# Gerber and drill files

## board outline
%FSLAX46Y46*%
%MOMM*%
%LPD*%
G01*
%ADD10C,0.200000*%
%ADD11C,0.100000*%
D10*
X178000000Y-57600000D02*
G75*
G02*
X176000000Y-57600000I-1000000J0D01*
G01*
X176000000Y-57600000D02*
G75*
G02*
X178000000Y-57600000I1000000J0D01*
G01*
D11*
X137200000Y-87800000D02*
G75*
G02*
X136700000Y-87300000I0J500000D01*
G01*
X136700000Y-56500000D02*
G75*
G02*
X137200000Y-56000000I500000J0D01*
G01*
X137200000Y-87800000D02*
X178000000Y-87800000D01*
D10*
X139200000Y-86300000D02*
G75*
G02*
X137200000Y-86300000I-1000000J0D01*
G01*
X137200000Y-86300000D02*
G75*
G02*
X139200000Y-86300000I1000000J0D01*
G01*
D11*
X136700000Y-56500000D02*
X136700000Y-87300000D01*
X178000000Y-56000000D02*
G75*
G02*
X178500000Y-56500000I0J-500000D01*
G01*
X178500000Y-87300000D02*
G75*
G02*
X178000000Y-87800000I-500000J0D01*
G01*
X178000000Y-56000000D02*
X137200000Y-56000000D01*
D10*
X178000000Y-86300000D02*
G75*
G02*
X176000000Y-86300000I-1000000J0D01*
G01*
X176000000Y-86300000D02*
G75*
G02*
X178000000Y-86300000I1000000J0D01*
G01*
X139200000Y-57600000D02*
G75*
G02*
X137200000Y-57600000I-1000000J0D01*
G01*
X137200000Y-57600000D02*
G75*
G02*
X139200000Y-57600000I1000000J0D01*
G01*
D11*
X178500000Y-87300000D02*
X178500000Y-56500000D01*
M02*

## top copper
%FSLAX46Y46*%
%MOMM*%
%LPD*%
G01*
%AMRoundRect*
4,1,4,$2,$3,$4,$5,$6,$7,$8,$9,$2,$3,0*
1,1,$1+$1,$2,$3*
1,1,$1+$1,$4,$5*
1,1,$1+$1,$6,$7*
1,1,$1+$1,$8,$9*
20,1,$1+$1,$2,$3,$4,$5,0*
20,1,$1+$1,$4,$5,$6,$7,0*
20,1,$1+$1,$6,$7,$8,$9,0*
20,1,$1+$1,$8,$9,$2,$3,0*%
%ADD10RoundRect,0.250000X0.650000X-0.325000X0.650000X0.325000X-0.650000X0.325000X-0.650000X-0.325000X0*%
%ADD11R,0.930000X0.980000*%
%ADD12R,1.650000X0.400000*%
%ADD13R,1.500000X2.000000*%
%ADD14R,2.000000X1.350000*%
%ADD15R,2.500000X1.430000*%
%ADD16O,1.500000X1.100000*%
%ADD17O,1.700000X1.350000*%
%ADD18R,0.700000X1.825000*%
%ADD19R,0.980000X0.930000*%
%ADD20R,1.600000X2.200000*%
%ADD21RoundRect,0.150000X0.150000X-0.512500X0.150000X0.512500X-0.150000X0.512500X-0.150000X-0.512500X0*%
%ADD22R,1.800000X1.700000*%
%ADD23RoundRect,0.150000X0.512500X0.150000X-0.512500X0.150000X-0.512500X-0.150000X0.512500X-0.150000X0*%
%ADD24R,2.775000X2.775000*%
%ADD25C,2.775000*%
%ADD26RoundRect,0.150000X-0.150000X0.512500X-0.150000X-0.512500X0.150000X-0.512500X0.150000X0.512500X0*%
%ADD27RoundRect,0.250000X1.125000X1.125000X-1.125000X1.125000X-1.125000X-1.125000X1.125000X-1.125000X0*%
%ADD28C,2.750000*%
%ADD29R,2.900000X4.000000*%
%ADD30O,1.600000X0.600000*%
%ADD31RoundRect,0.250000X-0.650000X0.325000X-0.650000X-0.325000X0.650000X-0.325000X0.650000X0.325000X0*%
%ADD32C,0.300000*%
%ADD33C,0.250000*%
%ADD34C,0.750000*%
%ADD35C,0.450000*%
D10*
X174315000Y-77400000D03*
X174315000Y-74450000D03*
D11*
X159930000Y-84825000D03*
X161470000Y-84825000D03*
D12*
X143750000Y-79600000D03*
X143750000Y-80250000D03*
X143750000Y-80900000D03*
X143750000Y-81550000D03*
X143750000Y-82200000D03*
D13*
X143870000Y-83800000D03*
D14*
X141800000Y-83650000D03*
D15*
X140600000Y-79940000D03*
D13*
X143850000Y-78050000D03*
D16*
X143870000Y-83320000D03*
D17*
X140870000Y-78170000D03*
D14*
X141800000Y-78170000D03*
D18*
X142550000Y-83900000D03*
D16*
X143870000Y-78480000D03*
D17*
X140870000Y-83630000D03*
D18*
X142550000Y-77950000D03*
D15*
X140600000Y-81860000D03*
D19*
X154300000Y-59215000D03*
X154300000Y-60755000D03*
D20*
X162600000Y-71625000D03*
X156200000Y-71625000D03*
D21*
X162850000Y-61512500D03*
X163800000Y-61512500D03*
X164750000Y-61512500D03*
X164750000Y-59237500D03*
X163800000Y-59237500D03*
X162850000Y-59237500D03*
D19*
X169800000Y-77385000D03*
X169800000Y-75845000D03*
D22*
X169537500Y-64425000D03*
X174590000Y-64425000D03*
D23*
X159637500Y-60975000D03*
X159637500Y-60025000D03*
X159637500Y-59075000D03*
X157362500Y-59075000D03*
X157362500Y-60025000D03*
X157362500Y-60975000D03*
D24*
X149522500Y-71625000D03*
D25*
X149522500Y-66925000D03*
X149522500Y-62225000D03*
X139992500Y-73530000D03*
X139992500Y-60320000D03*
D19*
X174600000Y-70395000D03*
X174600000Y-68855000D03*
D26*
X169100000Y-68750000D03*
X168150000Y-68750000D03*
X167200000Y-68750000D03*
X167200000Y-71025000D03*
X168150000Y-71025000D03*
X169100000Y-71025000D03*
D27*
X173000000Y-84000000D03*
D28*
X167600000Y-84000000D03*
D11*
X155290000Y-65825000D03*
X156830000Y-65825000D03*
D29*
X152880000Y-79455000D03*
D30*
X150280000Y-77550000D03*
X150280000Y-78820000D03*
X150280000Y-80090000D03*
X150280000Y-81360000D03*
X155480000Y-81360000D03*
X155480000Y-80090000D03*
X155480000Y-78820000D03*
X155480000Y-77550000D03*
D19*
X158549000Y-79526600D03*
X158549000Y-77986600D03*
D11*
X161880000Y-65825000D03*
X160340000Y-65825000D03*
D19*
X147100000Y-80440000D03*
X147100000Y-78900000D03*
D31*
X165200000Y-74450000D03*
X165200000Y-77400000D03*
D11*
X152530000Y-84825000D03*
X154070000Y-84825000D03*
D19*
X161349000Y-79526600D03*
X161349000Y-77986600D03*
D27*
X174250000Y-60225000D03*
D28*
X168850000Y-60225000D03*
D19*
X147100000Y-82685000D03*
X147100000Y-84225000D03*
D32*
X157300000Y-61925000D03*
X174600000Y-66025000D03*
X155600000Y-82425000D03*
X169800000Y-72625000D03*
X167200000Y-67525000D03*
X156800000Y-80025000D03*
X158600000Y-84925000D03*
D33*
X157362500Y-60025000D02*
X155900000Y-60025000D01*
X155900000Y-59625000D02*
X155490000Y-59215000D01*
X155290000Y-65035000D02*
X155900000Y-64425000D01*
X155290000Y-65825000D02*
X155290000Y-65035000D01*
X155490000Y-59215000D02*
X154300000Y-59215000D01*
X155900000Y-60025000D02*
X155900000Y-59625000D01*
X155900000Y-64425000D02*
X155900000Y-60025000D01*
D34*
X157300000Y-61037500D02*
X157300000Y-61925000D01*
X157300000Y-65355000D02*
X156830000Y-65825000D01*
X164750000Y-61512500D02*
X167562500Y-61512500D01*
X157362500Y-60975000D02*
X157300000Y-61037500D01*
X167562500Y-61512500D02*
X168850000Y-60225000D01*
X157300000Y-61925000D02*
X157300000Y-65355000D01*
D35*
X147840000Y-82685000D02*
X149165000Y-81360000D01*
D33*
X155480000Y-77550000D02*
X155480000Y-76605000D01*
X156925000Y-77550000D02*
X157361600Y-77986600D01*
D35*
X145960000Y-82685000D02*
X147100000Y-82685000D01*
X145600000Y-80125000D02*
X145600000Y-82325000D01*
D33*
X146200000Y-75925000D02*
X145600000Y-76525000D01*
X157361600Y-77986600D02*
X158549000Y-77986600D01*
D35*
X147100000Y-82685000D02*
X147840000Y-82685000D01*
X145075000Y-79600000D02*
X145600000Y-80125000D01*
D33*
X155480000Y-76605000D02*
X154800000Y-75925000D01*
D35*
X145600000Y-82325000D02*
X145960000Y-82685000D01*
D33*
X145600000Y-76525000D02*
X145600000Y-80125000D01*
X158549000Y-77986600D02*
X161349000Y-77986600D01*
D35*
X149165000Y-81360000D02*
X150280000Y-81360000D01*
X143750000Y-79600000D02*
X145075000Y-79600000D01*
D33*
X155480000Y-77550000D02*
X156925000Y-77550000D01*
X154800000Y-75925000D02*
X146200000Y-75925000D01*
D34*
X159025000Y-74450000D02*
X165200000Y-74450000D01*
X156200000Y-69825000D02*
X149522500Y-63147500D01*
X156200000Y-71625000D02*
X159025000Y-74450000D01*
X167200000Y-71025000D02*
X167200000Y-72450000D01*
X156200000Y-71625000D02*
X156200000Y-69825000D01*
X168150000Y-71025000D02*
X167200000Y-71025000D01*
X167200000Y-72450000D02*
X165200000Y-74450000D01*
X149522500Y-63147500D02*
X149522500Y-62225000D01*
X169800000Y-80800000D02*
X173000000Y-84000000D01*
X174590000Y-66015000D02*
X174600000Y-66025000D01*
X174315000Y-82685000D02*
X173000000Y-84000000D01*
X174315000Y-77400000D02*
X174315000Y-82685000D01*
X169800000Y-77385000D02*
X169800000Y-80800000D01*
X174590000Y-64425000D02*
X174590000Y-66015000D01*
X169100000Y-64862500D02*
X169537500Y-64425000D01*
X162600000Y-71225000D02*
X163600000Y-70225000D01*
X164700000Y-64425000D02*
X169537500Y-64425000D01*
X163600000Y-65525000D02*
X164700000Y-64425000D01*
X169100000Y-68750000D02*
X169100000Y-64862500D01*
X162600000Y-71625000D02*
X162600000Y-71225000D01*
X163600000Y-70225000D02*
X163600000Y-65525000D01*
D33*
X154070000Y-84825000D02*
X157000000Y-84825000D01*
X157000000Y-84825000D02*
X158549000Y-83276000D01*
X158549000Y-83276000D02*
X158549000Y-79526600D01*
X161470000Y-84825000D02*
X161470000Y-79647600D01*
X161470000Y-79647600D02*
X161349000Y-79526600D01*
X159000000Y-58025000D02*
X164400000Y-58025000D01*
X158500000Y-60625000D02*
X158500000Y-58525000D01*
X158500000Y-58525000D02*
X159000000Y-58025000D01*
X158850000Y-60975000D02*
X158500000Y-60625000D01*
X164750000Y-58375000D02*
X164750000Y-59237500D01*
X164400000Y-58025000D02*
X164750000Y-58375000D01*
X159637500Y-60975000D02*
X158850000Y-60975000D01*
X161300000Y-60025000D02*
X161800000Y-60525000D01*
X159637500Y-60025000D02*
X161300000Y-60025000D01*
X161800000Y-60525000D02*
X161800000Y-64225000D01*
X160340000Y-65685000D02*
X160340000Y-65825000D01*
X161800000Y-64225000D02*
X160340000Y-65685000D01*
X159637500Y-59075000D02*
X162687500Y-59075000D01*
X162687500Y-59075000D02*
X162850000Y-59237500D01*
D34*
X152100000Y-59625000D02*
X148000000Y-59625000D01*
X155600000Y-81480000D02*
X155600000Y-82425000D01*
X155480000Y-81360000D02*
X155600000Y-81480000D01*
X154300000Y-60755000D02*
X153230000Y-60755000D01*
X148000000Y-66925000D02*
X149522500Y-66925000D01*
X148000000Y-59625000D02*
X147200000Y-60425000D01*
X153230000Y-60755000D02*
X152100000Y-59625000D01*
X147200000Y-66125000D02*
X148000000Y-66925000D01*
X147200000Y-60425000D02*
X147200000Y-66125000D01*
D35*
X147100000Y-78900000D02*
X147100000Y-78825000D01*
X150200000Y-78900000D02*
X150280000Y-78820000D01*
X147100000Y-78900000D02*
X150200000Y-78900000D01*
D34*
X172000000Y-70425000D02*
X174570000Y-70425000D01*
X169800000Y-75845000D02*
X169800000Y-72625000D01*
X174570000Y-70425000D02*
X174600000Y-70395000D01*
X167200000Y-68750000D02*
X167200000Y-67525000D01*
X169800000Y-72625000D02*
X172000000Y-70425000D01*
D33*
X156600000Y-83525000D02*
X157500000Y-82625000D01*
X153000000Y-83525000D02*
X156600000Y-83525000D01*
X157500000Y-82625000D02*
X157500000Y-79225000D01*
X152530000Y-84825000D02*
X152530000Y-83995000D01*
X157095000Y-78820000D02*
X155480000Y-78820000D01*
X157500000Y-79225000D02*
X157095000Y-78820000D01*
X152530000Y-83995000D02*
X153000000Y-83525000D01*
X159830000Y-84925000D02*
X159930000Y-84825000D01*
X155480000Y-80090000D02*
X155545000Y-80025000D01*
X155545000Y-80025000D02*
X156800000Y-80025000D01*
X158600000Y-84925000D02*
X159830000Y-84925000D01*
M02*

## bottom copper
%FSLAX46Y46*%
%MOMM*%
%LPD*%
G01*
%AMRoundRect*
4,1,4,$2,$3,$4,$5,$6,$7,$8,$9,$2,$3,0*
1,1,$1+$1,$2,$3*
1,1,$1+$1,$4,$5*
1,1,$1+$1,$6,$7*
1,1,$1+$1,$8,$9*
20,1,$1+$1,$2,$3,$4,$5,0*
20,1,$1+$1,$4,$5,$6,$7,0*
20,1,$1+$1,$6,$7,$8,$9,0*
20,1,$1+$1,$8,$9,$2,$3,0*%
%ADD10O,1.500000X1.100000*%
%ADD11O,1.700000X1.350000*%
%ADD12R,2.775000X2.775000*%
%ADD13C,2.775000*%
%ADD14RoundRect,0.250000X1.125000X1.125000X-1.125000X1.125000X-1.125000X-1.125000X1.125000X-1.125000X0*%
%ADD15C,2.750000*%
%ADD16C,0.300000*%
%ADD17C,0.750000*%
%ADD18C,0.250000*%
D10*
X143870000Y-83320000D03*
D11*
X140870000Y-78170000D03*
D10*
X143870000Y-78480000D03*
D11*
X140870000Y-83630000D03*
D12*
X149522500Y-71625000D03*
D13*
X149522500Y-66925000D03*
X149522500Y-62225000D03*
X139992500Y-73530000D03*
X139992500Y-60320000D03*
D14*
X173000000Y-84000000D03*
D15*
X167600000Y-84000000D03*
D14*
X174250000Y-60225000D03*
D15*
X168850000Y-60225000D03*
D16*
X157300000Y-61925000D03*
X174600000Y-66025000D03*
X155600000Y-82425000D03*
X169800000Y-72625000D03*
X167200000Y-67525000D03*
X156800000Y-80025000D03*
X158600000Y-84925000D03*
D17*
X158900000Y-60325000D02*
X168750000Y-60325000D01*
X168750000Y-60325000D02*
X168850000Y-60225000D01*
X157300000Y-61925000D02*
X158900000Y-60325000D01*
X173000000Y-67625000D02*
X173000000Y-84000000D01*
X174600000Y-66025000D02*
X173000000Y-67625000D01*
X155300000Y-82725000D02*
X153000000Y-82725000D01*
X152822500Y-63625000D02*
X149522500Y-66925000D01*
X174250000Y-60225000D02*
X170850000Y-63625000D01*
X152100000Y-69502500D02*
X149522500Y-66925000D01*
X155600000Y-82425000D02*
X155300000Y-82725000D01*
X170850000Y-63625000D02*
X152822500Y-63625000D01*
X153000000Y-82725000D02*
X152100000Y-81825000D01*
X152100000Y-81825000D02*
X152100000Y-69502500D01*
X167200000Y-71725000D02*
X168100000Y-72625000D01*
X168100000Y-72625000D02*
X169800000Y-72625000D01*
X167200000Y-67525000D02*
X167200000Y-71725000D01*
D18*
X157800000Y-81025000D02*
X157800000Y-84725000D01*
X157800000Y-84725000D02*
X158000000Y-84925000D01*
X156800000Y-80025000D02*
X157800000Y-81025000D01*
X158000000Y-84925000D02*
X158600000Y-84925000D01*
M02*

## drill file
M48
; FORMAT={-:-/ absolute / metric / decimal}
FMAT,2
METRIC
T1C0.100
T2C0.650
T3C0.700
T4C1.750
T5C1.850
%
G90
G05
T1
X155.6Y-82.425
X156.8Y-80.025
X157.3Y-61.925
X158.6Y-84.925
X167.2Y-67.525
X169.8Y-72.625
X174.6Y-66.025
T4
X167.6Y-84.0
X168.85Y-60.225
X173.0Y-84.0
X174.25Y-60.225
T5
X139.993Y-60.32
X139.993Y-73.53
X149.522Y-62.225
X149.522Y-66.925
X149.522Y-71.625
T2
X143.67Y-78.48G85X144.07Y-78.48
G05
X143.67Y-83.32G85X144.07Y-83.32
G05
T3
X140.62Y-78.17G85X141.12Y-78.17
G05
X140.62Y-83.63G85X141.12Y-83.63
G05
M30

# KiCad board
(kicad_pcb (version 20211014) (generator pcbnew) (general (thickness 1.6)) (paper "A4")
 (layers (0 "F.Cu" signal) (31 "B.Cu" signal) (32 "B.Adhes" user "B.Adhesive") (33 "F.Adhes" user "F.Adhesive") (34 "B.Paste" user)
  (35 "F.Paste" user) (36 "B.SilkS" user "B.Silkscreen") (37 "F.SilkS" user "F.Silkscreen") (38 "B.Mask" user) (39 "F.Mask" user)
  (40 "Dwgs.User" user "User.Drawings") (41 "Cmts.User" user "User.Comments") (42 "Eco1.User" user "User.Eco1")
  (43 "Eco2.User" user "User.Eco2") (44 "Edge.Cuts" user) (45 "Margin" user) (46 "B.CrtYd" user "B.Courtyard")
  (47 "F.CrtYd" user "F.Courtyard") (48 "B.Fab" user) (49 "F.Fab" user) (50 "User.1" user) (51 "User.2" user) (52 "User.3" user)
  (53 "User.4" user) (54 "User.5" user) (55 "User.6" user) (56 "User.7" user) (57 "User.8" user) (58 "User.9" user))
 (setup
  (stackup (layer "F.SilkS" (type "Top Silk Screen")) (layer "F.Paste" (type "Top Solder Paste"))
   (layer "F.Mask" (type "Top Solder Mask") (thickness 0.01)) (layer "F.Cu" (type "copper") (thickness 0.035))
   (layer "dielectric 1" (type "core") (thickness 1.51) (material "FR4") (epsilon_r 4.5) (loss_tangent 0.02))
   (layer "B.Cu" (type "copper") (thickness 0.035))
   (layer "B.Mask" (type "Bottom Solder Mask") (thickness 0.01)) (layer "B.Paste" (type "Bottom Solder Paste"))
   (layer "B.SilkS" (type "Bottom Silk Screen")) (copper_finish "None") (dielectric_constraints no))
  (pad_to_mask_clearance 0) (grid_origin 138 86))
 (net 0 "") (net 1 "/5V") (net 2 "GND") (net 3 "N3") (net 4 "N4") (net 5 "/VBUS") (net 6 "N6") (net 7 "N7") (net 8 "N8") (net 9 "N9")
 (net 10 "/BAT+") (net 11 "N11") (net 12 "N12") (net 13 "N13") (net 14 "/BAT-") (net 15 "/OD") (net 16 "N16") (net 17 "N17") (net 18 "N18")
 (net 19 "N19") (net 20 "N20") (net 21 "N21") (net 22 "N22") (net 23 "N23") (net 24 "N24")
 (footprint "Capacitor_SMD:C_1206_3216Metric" (layer "F.Cu") (at 174.315 75.925 90)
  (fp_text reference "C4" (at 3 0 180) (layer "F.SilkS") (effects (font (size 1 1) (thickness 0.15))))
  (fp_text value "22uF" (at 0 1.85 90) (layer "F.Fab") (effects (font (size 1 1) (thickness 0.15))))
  (pad "1" smd roundrect (at -1.475 0 90) (size 1.15 1.8) (layers "F.Cu" "F.Paste" "F.Mask") (roundrect_rratio 0.217391) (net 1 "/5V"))
  (pad "2" smd roundrect (at 1.475 0 90) (size 1.15 1.8) (layers "F.Cu" "F.Paste" "F.Mask") (roundrect_rratio 0.217391) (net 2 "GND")))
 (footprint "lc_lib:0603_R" (layer "F.Cu") (at 160.7 84.825)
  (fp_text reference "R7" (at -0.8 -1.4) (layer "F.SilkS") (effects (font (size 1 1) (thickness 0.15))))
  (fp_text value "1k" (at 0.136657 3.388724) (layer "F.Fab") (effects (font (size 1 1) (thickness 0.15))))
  (pad "1" smd rect locked (at -0.77 0) (size 0.93 0.98) (layers "F.Cu" "F.Paste" "F.Mask") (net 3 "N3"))
  (pad "2" smd rect locked (at 0.77 0) (size 0.93 0.98) (layers "F.Cu" "F.Paste" "F.Mask") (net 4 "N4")))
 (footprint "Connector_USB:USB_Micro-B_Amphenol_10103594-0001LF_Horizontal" (layer "F.Cu") (at 141.985 80.925 -90)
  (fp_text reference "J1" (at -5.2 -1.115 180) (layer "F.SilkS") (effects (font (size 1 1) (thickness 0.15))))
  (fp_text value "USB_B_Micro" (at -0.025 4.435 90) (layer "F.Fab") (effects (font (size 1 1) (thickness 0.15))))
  (pad "1" smd rect (at -1.325 -1.765) (size 1.65 0.4) (layers "F.Cu" "F.Paste" "F.Mask") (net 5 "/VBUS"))
  (pad "2" smd rect (at -0.675 -1.765) (size 1.65 0.4) (layers "F.Cu" "F.Paste" "F.Mask") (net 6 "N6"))
  (pad "3" smd rect (at -0.025 -1.765) (size 1.65 0.4) (layers "F.Cu" "F.Paste" "F.Mask") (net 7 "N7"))
  (pad "4" smd rect (at 0.625 -1.765) (size 1.65 0.4) (layers "F.Cu" "F.Paste" "F.Mask") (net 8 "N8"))
  (pad "5" smd rect (at 1.275 -1.765) (size 1.65 0.4) (layers "F.Cu" "F.Paste" "F.Mask") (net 2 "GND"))
  (pad "6" smd rect (at 2.875 -1.885 270) (size 2 1.5) (layers "F.Cu" "F.Paste" "F.Mask") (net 2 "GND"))
  (pad "6" smd rect (at 2.725 0.185 270) (size 1.35 2) (layers "F.Cu" "F.Paste" "F.Mask") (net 2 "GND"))
  (pad "6" smd rect (at -0.985 1.385) (size 2.5 1.43) (layers "F.Cu" "F.Paste" "F.Mask") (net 2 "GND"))
  (pad "6" smd rect (at -2.875 -1.865 270) (size 2 1.5) (layers "F.Cu" "F.Paste" "F.Mask") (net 2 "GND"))
  (pad "6" thru_hole oval (at 2.395 -1.885) (size 1.5 1.1) (drill oval 1.05 0.65) (layers *.Cu *.Mask) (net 2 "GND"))
  (pad "6" thru_hole oval (at -2.755 1.115) (size 1.7 1.35) (drill oval 1.2 0.7) (layers *.Cu *.Mask) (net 2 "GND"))
  (pad "6" smd rect (at -2.755 0.185 270) (size 1.35 2) (layers "F.Cu" "F.Paste" "F.Mask") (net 2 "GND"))
  (pad "6" smd rect (at 2.975 -0.565 270) (size 1.825 0.7) (layers "F.Cu" "F.Paste" "F.Mask") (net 2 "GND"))
  (pad "6" thru_hole oval (at -2.445 -1.885) (size 1.5 1.1) (drill oval 1.05 0.65) (layers *.Cu *.Mask) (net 2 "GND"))
  (pad "6" thru_hole oval (at 2.705 1.115) (size 1.7 1.35) (drill oval 1.2 0.7) (layers *.Cu *.Mask) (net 2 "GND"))
  (pad "6" smd rect (at -2.975 -0.565 270) (size 1.825 0.7) (layers "F.Cu" "F.Paste" "F.Mask") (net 2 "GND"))
  (pad "6" smd rect (at 0.935 1.385) (size 2.5 1.43) (layers "F.Cu" "F.Paste" "F.Mask") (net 2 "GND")))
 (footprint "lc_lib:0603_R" (layer "F.Cu") (at 154.3 59.985 -90)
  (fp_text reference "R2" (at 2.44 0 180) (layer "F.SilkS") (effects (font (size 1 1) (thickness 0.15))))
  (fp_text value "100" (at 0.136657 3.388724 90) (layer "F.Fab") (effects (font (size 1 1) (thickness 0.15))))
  (pad "1" smd rect locked (at -0.77 0 270) (size 0.93 0.98) (layers "F.Cu" "F.Paste" "F.Mask") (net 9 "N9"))
  (pad "2" smd rect locked (at 0.77 0 270) (size 0.93 0.98) (layers "F.Cu" "F.Paste" "F.Mask") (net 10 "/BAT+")))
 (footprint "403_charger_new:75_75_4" (layer "F.Cu") (at 163.15 67.625 180)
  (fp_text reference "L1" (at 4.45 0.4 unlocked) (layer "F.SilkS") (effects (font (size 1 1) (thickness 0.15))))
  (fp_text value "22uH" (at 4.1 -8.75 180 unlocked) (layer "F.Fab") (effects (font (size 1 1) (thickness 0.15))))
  (pad "1" smd rect (at 0.55 -4 90) (size 2.2 1.6) (layers "F.Cu" "F.Paste" "F.Mask") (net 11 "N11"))
  (pad "2" smd rect (at 6.95 -4 90) (size 2.2 1.6) (layers "F.Cu" "F.Adhes" "F.Paste" "F.Mask") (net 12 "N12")))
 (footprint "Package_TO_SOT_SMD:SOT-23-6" (layer "F.Cu") (at 163.8 60.375 90)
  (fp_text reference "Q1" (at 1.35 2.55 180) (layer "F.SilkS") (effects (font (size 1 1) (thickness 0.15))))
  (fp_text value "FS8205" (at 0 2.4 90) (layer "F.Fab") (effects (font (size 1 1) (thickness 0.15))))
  (pad "1" smd roundrect (at -1.1375 -0.95 90) (size 1.325 0.6) (layers "F.Cu" "F.Paste" "F.Mask") (roundrect_rratio 0.25) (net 2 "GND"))
  (pad "2" smd roundrect (at -1.1375 0 90) (size 1.325 0.6) (layers "F.Cu" "F.Paste" "F.Mask") (roundrect_rratio 0.25) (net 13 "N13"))
  (pad "3" smd roundrect (at -1.1375 0.95 90) (size 1.325 0.6) (layers "F.Cu" "F.Paste" "F.Mask") (roundrect_rratio 0.25) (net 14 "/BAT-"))
  (pad "4" smd roundrect (at 1.1375 0.95 90) (size 1.325 0.6) (layers "F.Cu" "F.Paste" "F.Mask") (roundrect_rratio 0.25) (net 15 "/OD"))
  (pad "5" smd roundrect (at 1.1375 0 90) (size 1.325 0.6) (layers "F.Cu" "F.Paste" "F.Mask") (roundrect_rratio 0.25) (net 13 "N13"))
  (pad "6" smd roundrect (at 1.1375 -0.95 90) (size 1.325 0.6) (layers "F.Cu" "F.Paste" "F.Mask") (roundrect_rratio 0.25) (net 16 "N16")))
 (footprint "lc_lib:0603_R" (layer "F.Cu") (at 169.8 76.615 90)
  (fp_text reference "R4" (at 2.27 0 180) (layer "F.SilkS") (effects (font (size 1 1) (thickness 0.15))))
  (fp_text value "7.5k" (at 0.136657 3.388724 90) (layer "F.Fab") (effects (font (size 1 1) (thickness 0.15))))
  (pad "1" smd rect locked (at -0.77 0 90) (size 0.93 0.98) (layers "F.Cu" "F.Paste" "F.Mask") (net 1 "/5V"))
  (pad "2" smd rect locked (at 0.77 0 90) (size 0.93 0.98) (layers "F.Cu" "F.Paste" "F.Mask") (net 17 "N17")))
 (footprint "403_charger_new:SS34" (layer "F.Cu") (at 172.06375 64.425 180)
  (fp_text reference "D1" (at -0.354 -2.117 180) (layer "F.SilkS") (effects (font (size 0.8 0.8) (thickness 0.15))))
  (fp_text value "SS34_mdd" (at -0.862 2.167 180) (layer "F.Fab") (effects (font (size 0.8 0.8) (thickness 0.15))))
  (pad "A" smd rect (at 2.52625 0 180) (size 1.8 1.7) (layers "F.Cu" "F.Paste" "F.Mask") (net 11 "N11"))
  (pad "C" smd rect (at -2.52625 0 180) (size 1.8 1.7) (layers "F.Cu" "F.Paste" "F.Mask") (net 1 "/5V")))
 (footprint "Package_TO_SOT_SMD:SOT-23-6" (layer "F.Cu") (at 158.5 60.025 180)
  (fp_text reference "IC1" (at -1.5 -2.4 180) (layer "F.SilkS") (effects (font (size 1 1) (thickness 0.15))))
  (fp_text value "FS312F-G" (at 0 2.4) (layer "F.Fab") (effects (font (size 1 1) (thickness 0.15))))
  (pad "1" smd roundrect (at -1.1375 -0.95 180) (size 1.325 0.6) (layers "F.Cu" "F.Paste" "F.Mask") (roundrect_rratio 0.25) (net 15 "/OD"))
  (pad "2" smd roundrect (at -1.1375 0 180) (size 1.325 0.6) (layers "F.Cu" "F.Paste" "F.Mask") (roundrect_rratio 0.25) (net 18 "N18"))
  (pad "3" smd roundrect (at -1.1375 0.95 180) (size 1.325 0.6) (layers "F.Cu" "F.Paste" "F.Mask") (roundrect_rratio 0.25) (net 16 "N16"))
  (pad "4" smd roundrect (at 1.1375 0.95 180) (size 1.325 0.6) (layers "F.Cu" "F.Paste" "F.Mask") (roundrect_rratio 0.25) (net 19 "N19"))
  (pad "5" smd roundrect (at 1.1375 0 180) (size 1.325 0.6) (layers "F.Cu" "F.Paste" "F.Mask") (roundrect_rratio 0.25) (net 9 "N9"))
  (pad "6" smd roundrect (at 1.1375 -0.95 180) (size 1.325 0.6) (layers "F.Cu" "F.Paste" "F.Mask") (roundrect_rratio 0.25) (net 14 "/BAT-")))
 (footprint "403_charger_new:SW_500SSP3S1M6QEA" (layer "F.Cu") (at 144.7575 66.925 90)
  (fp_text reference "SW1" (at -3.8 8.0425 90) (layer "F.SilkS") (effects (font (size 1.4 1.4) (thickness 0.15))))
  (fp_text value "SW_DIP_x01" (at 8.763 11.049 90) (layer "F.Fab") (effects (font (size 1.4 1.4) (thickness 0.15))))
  (pad "1" thru_hole rect (at -4.7 4.765 90) (size 2.775 2.775) (drill 1.85) (layers *.Cu *.Mask) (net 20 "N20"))
  (pad "2" thru_hole circle (at 0 4.765 90) (size 2.775 2.775) (drill 1.85) (layers *.Cu *.Mask) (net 10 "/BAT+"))
  (pad "3" thru_hole circle (at 4.7 4.765 90) (size 2.775 2.775) (drill 1.85) (layers *.Cu *.Mask) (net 12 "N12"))
  (pad "S1" thru_hole circle (at -6.605 -4.765 90) (size 2.775 2.775) (drill 1.85) (layers *.Cu *.Mask))
  (pad "S2" thru_hole circle (at 6.605 -4.765 90) (size 2.775 2.775) (drill 1.85) (layers *.Cu *.Mask)))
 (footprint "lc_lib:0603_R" (layer "F.Cu") (at 174.6 69.625 90)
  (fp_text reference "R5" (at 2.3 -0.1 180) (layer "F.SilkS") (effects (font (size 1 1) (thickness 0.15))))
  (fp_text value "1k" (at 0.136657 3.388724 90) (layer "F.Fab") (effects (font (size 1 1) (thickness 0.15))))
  (pad "1" smd rect locked (at -0.77 0 90) (size 0.93 0.98) (layers "F.Cu" "F.Paste" "F.Mask") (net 17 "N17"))
  (pad "2" smd rect locked (at 0.77 0 90) (size 0.93 0.98) (layers "F.Cu" "F.Paste" "F.Mask") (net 2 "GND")))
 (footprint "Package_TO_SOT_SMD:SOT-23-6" (layer "F.Cu") (at 168.15 69.8875 -90)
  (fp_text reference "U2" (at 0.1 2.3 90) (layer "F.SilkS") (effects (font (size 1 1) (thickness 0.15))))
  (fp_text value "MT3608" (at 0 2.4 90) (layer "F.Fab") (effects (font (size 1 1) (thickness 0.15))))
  (pad "1" smd roundrect (at -1.1375 -0.95 270) (size 1.325 0.6) (layers "F.Cu" "F.Paste" "F.Mask") (roundrect_rratio 0.25) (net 11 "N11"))
  (pad "2" smd roundrect (at -1.1375 0 270) (size 1.325 0.6) (layers "F.Cu" "F.Paste" "F.Mask") (roundrect_rratio 0.25) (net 2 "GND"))
  (pad "3" smd roundrect (at -1.1375 0.95 270) (size 1.325 0.6) (layers "F.Cu" "F.Paste" "F.Mask") (roundrect_rratio 0.25) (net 17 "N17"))
  (pad "4" smd roundrect (at 1.1375 0.95 270) (size 1.325 0.6) (layers "F.Cu" "F.Paste" "F.Mask") (roundrect_rratio 0.25) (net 12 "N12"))
  (pad "5" smd roundrect (at 1.1375 0 270) (size 1.325 0.6) (layers "F.Cu" "F.Paste" "F.Mask") (roundrect_rratio 0.25) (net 12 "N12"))
  (pad "6" smd roundrect (at 1.1375 -0.95 270) (size 1.325 0.6) (layers "F.Cu" "F.Paste" "F.Mask") (roundrect_rratio 0.25) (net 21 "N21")))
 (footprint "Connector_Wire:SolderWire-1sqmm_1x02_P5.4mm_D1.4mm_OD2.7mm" (layer "F.Cu") (at 173 84 180)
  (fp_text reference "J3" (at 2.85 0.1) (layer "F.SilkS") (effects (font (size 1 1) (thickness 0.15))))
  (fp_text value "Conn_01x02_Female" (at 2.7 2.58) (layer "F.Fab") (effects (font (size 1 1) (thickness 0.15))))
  (pad "1" thru_hole roundrect (at 0 0 180) (size 2.75 2.75) (drill 1.75) (layers *.Cu *.Mask) (roundrect_rratio 0.090909) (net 1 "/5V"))
  (pad "2" thru_hole circle (at 5.4 0 180) (size 2.75 2.75) (drill 1.75) (layers *.Cu *.Mask) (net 2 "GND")))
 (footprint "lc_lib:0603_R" (layer "F.Cu") (at 156.06 65.825)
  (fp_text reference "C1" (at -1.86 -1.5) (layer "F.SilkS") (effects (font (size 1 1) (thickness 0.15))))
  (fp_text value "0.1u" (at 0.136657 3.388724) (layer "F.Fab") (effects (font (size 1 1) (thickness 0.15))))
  (pad "1" smd rect locked (at -0.77 0) (size 0.93 0.98) (layers "F.Cu" "F.Paste" "F.Mask") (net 9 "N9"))
  (pad "2" smd rect locked (at 0.77 0) (size 0.93 0.98) (layers "F.Cu" "F.Paste" "F.Mask") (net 14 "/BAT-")))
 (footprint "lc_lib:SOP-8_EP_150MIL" (layer "F.Cu") (at 152.88 79.455 -90)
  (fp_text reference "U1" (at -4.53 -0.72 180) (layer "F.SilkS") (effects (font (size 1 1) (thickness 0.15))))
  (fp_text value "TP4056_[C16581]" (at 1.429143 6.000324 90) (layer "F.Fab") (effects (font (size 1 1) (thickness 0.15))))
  (pad "0" smd rect (at 0 0 90) (size 4 2.9) (layers "F.Cu" "F.Paste" "F.Mask"))
  (pad "1" smd oval (at -1.905 2.6 90) (size 0.6 1.6) (layers "F.Cu" "F.Paste" "F.Mask") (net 2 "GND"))
  (pad "2" smd oval (at -0.635 2.6 90) (size 0.6 1.6) (layers "F.Cu" "F.Paste" "F.Mask") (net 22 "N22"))
  (pad "3" smd oval (at 0.635 2.6 90) (size 0.6 1.6) (layers "F.Cu" "F.Paste" "F.Mask") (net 2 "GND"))
  (pad "4" smd oval (at 1.905 2.6 90) (size 0.6 1.6) (layers "F.Cu" "F.Paste" "F.Mask") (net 5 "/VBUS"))
  (pad "5" smd oval (at 1.905 -2.6 90) (size 0.6 1.6) (layers "F.Cu" "F.Paste" "F.Mask") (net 10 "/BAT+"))
  (pad "6" smd oval (at 0.635 -2.6 90) (size 0.6 1.6) (layers "F.Cu" "F.Paste" "F.Mask") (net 3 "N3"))
  (pad "7" smd oval (at -0.635 -2.6 90) (size 0.6 1.6) (layers "F.Cu" "F.Paste" "F.Mask") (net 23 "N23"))
  (pad "8" smd oval (at -1.905 -2.6 90) (size 0.6 1.6) (layers "F.Cu" "F.Paste" "F.Mask") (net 5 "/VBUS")))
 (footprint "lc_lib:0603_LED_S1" (layer "F.Cu") (at 158.549 78.7566 -90)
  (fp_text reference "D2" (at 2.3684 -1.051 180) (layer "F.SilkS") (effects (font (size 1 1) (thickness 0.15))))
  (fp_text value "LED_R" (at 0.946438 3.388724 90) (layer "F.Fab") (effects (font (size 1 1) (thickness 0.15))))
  (pad "1" smd rect (at 0.77 0 90) (size 0.93 0.98) (layers "F.Cu" "F.Paste" "F.Mask") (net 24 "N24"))
  (pad "2" smd rect (at -0.77 0 90) (size 0.93 0.98) (layers "F.Cu" "F.Paste" "F.Mask") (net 5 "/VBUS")))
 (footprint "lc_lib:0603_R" (layer "F.Cu") (at 161.11 65.825 180)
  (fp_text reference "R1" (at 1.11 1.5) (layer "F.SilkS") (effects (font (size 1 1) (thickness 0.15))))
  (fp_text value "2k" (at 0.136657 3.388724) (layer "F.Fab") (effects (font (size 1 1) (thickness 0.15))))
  (pad "1" smd rect locked (at -0.77 0 180) (size 0.93 0.98) (layers "F.Cu" "F.Paste" "F.Mask") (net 2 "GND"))
  (pad "2" smd rect locked (at 0.77 0 180) (size 0.93 0.98) (layers "F.Cu" "F.Paste" "F.Mask") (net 18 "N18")))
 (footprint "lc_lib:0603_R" (layer "F.Cu") (at 147.1 79.67 90)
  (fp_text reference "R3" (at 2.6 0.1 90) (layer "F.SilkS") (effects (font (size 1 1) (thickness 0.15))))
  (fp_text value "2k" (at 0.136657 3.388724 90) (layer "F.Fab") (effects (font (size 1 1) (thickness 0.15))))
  (pad "1" smd rect locked (at -0.77 0 90) (size 0.93 0.98) (layers "F.Cu" "F.Paste" "F.Mask") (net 2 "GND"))
  (pad "2" smd rect locked (at 0.77 0 90) (size 0.93 0.98) (layers "F.Cu" "F.Paste" "F.Mask") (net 22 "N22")))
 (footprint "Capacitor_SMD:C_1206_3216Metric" (layer "F.Cu") (at 165.2 75.925 -90)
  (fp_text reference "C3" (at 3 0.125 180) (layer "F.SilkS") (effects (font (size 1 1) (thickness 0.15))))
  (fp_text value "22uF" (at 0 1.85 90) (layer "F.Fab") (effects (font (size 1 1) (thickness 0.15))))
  (pad "1" smd roundrect (at -1.475 0 270) (size 1.15 1.8) (layers "F.Cu" "F.Paste" "F.Mask") (roundrect_rratio 0.217391) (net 12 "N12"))
  (pad "2" smd roundrect (at 1.475 0 270) (size 1.15 1.8) (layers "F.Cu" "F.Paste" "F.Mask") (roundrect_rratio 0.217391) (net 2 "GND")))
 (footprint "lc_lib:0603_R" (layer "F.Cu") (at 153.3 84.825)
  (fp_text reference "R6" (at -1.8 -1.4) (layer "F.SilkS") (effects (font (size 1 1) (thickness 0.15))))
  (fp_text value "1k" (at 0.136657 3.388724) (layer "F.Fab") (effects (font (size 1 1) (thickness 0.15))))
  (pad "1" smd rect locked (at -0.77 0) (size 0.93 0.98) (layers "F.Cu" "F.Paste" "F.Mask") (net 23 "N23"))
  (pad "2" smd rect locked (at 0.77 0) (size 0.93 0.98) (layers "F.Cu" "F.Paste" "F.Mask") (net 24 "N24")))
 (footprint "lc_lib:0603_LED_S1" (layer "F.Cu") (at 161.349 78.7566 -90)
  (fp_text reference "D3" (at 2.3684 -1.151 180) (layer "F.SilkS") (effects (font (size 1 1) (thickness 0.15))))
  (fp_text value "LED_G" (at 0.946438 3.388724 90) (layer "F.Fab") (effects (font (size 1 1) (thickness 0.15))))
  (pad "1" smd rect (at 0.77 0 90) (size 0.93 0.98) (layers "F.Cu" "F.Paste" "F.Mask") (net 4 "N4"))
  (pad "2" smd rect (at -0.77 0 90) (size 0.93 0.98) (layers "F.Cu" "F.Paste" "F.Mask") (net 5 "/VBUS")))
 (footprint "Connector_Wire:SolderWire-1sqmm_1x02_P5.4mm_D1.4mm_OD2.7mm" (layer "F.Cu") (at 174.25 60.225 180)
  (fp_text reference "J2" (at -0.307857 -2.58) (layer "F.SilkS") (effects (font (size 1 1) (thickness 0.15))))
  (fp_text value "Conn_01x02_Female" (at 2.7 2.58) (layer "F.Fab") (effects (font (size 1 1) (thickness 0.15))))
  (pad "1" thru_hole roundrect (at 0 0 180) (size 2.75 2.75) (drill 1.75) (layers *.Cu *.Mask) (roundrect_rratio 0.090909) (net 10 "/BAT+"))
  (pad "2" thru_hole circle (at 5.4 0 180) (size 2.75 2.75) (drill 1.75) (layers *.Cu *.Mask) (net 14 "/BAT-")))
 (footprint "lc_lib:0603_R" (layer "F.Cu") (at 147.1 83.455 -90)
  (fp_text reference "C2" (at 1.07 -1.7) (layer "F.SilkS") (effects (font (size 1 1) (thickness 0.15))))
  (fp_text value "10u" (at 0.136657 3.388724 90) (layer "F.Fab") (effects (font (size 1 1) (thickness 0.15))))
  (pad "1" smd rect locked (at -0.77 0 270) (size 0.93 0.98) (layers "F.Cu" "F.Paste" "F.Mask") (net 5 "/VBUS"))
  (pad "2" smd rect locked (at 0.77 0 270) (size 0.93 0.98) (layers "F.Cu" "F.Paste" "F.Mask") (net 2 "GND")))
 (gr_circle (center 177 57.6) (end 178 57.6) (layer "Edge.Cuts") (width 0.2) (fill none))
 (gr_arc (start 137.2 87.8) (mid 136.846447 87.653553) (end 136.7 87.3) (layer "Edge.Cuts") (width 0.1))
 (gr_arc (start 136.7 56.5) (mid 136.846447 56.146447) (end 137.2 56) (layer "Edge.Cuts") (width 0.1))
 (gr_line (start 137.2 87.8) (end 178 87.8) (layer "Edge.Cuts") (width 0.1))
 (gr_circle (center 138.2 86.3) (end 138.2 85.3) (layer "Edge.Cuts") (width 0.2) (fill none))
 (gr_line (start 136.7 56.5) (end 136.7 87.3) (layer "Edge.Cuts") (width 0.1))
 (gr_arc (start 178 56) (mid 178.353553 56.146447) (end 178.5 56.5) (layer "Edge.Cuts") (width 0.1))
 (gr_arc (start 178.5 87.3) (mid 178.353553 87.653553) (end 178 87.8) (layer "Edge.Cuts") (width 0.1))
 (gr_line (start 178 56) (end 137.2 56) (layer "Edge.Cuts") (width 0.1))
 (gr_circle (center 177 86.3) (end 177 85.3) (layer "Edge.Cuts") (width 0.2) (fill none))
 (gr_circle (center 138.2 57.6) (end 138.2 56.6) (layer "Edge.Cuts") (width 0.2) (fill none))
 (gr_line (start 178.5 87.3) (end 178.5 56.5) (layer "Edge.Cuts") (width 0.1))
 (segment (start 157.3625 60.025) (end 155.9 60.025) (width 0.25) (layer "F.Cu") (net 9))
 (segment (start 155.9 59.625) (end 155.49 59.215) (width 0.25) (layer "F.Cu") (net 9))
 (segment (start 155.29 65.035) (end 155.9 64.425) (width 0.25) (layer "F.Cu") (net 9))
 (segment (start 155.29 65.825) (end 155.29 65.035) (width 0.25) (layer "F.Cu") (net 9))
 (segment (start 155.49 59.215) (end 154.3 59.215) (width 0.25) (layer "F.Cu") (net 9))
 (segment (start 155.9 60.025) (end 155.9 59.625) (width 0.25) (layer "F.Cu") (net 9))
 (segment (start 155.9 64.425) (end 155.9 60.025) (width 0.25) (layer "F.Cu") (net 9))
 (segment (start 157.3 61.0375) (end 157.3 61.925) (width 0.75) (layer "F.Cu") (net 14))
 (segment (start 157.3 65.355) (end 156.83 65.825) (width 0.75) (layer "F.Cu") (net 14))
 (segment (start 164.75 61.5125) (end 167.5625 61.5125) (width 0.75) (layer "F.Cu") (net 14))
 (segment (start 157.3625 60.975) (end 157.3 61.0375) (width 0.75) (layer "F.Cu") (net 14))
 (segment (start 167.5625 61.5125) (end 168.85 60.225) (width 0.75) (layer "F.Cu") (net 14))
 (segment (start 157.3 61.925) (end 157.3 65.355) (width 0.75) (layer "F.Cu") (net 14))
 (via micro (at 157.3 61.925) (size 0.3) (drill 0.1) (layers "F.Cu" "B.Cu") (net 14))
 (segment (start 158.9 60.325) (end 168.75 60.325) (width 0.75) (layer "B.Cu") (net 14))
 (segment (start 168.75 60.325) (end 168.85 60.225) (width 0.75) (layer "B.Cu") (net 14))
 (segment (start 157.3 61.925) (end 158.9 60.325) (width 0.75) (layer "B.Cu") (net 14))
 (segment (start 147.84 82.685) (end 149.165 81.36) (width 0.45) (layer "F.Cu") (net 5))
 (segment (start 155.48 77.55) (end 155.48 76.605) (width 0.25) (layer "F.Cu") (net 5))
 (segment (start 156.925 77.55) (end 157.3616 77.9866) (width 0.25) (layer "F.Cu") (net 5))
 (segment (start 145.96 82.685) (end 147.1 82.685) (width 0.45) (layer "F.Cu") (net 5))
 (segment (start 145.6 80.125) (end 145.6 82.325) (width 0.45) (layer "F.Cu") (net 5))
 (segment (start 146.2 75.925) (end 145.6 76.525) (width 0.25) (layer "F.Cu") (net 5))
 (segment (start 157.3616 77.9866) (end 158.549 77.9866) (width 0.25) (layer "F.Cu") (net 5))
 (segment (start 147.1 82.685) (end 147.84 82.685) (width 0.45) (layer "F.Cu") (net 5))
 (segment (start 145.075 79.6) (end 145.6 80.125) (width 0.45) (layer "F.Cu") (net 5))
 (segment (start 155.48 76.605) (end 154.8 75.925) (width 0.25) (layer "F.Cu") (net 5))
 (segment (start 145.6 82.325) (end 145.96 82.685) (width 0.45) (layer "F.Cu") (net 5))
 (segment (start 145.6 76.525) (end 145.6 80.125) (width 0.25) (layer "F.Cu") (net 5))
 (segment (start 158.549 77.9866) (end 161.349 77.9866) (width 0.25) (layer "F.Cu") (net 5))
 (segment (start 149.165 81.36) (end 150.28 81.36) (width 0.45) (layer "F.Cu") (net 5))
 (segment (start 143.75 79.6) (end 145.075 79.6) (width 0.45) (layer "F.Cu") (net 5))
 (segment (start 155.48 77.55) (end 156.925 77.55) (width 0.25) (layer "F.Cu") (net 5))
 (segment (start 154.8 75.925) (end 146.2 75.925) (width 0.25) (layer "F.Cu") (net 5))
 (segment (start 159.025 74.45) (end 165.2 74.45) (width 0.75) (layer "F.Cu") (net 12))
 (segment (start 156.2 69.825) (end 149.5225 63.1475) (width 0.75) (layer "F.Cu") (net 12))
 (segment (start 156.2 71.625) (end 159.025 74.45) (width 0.75) (layer "F.Cu") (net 12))
 (segment (start 167.2 71.025) (end 167.2 72.45) (width 0.75) (layer "F.Cu") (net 12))
 (segment (start 156.2 71.625) (end 156.2 69.825) (width 0.75) (layer "F.Cu") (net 12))
 (segment (start 168.15 71.025) (end 167.2 71.025) (width 0.75) (layer "F.Cu") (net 12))
 (segment (start 167.2 72.45) (end 165.2 74.45) (width 0.75) (layer "F.Cu") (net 12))
 (segment (start 149.5225 63.1475) (end 149.5225 62.225) (width 0.75) (layer "F.Cu") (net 12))
 (segment (start 169.8 80.8) (end 173 84) (width 0.75) (layer "F.Cu") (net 1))
 (segment (start 174.59 66.015) (end 174.6 66.025) (width 0.75) (layer "F.Cu") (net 1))
 (segment (start 174.315 82.685) (end 173 84) (width 0.75) (layer "F.Cu") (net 1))
 (segment (start 174.315 77.4) (end 174.315 82.685) (width 0.75) (layer "F.Cu") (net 1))
 (segment (start 169.8 77.385) (end 169.8 80.8) (width 0.75) (layer "F.Cu") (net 1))
 (segment (start 174.59 64.425) (end 174.59 66.015) (width 0.75) (layer "F.Cu") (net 1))
 (via micro (at 174.6 66.025) (size 0.3) (drill 0.1) (layers "F.Cu" "B.Cu") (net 1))
 (segment (start 173 67.625) (end 173 84) (width 0.75) (layer "B.Cu") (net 1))
 (segment (start 174.6 66.025) (end 173 67.625) (width 0.75) (layer "B.Cu") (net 1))
 (segment (start 169.1 64.8625) (end 169.5375 64.425) (width 0.75) (layer "F.Cu") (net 11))
 (segment (start 162.6 71.225) (end 163.6 70.225) (width 0.75) (layer "F.Cu") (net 11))
 (segment (start 164.7 64.425) (end 169.5375 64.425) (width 0.75) (layer "F.Cu") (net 11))
 (segment (start 163.6 65.525) (end 164.7 64.425) (width 0.75) (layer "F.Cu") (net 11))
 (segment (start 169.1 68.75) (end 169.1 64.8625) (width 0.75) (layer "F.Cu") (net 11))
 (segment (start 162.6 71.625) (end 162.6 71.225) (width 0.75) (layer "F.Cu") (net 11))
 (segment (start 163.6 70.225) (end 163.6 65.525) (width 0.75) (layer "F.Cu") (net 11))
 (segment (start 154.07 84.825) (end 157 84.825) (width 0.25) (layer "F.Cu") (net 24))
 (segment (start 157 84.825) (end 158.549 83.276) (width 0.25) (layer "F.Cu") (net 24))
 (segment (start 158.549 83.276) (end 158.549 79.5266) (width 0.25) (layer "F.Cu") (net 24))
 (segment (start 161.47 84.825) (end 161.47 79.6476) (width 0.25) (layer "F.Cu") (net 4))
 (segment (start 161.47 79.6476) (end 161.349 79.5266) (width 0.25) (layer "F.Cu") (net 4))
 (segment (start 159 58.025) (end 164.4 58.025) (width 0.25) (layer "F.Cu") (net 15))
 (segment (start 158.5 60.625) (end 158.5 58.525) (width 0.25) (layer "F.Cu") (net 15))
 (segment (start 158.5 58.525) (end 159 58.025) (width 0.25) (layer "F.Cu") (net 15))
 (segment (start 158.85 60.975) (end 158.5 60.625) (width 0.25) (layer "F.Cu") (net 15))
 (segment (start 164.75 58.375) (end 164.75 59.2375) (width 0.25) (layer "F.Cu") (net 15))
 (segment (start 164.4 58.025) (end 164.75 58.375) (width 0.25) (layer "F.Cu") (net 15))
 (segment (start 159.6375 60.975) (end 158.85 60.975) (width 0.25) (layer "F.Cu") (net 15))
 (segment (start 161.3 60.025) (end 161.8 60.525) (width 0.25) (layer "F.Cu") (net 18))
 (segment (start 159.6375 60.025) (end 161.3 60.025) (width 0.25) (layer "F.Cu") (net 18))
 (segment (start 161.8 60.525) (end 161.8 64.225) (width 0.25) (layer "F.Cu") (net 18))
 (segment (start 160.34 65.685) (end 160.34 65.825) (width 0.25) (layer "F.Cu") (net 18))
 (segment (start 161.8 64.225) (end 160.34 65.685) (width 0.25) (layer "F.Cu") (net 18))
 (segment (start 159.6375 59.075) (end 162.6875 59.075) (width 0.25) (layer "F.Cu") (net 16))
 (segment (start 162.6875 59.075) (end 162.85 59.2375) (width 0.25) (layer "F.Cu") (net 16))
 (segment (start 152.1 59.625) (end 148 59.625) (width 0.75) (layer "F.Cu") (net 10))
 (segment (start 155.6 81.48) (end 155.6 82.425) (width 0.75) (layer "F.Cu") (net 10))
 (segment (start 155.48 81.36) (end 155.6 81.48) (width 0.75) (layer "F.Cu") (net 10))
 (segment (start 154.3 60.755) (end 153.23 60.755) (width 0.75) (layer "F.Cu") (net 10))
 (segment (start 148 66.925) (end 149.5225 66.925) (width 0.75) (layer "F.Cu") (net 10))
 (segment (start 148 59.625) (end 147.2 60.425) (width 0.75) (layer "F.Cu") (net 10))
 (segment (start 153.23 60.755) (end 152.1 59.625) (width 0.75) (layer "F.Cu") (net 10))
 (segment (start 147.2 66.125) (end 148 66.925) (width 0.75) (layer "F.Cu") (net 10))
 (segment (start 147.2 60.425) (end 147.2 66.125) (width 0.75) (layer "F.Cu") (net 10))
 (via micro (at 155.6 82.425) (size 0.3) (drill 0.1) (layers "F.Cu" "B.Cu") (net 10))
 (segment (start 155.3 82.725) (end 153 82.725) (width 0.75) (layer "B.Cu") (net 10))
 (segment (start 152.8225 63.625) (end 149.5225 66.925) (width 0.75) (layer "B.Cu") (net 10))
 (segment (start 174.25 60.225) (end 170.85 63.625) (width 0.75) (layer "B.Cu") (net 10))
 (segment (start 152.1 69.5025) (end 149.5225 66.925) (width 0.75) (layer "B.Cu") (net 10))
 (segment (start 155.6 82.425) (end 155.3 82.725) (width 0.75) (layer "B.Cu") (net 10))
 (segment (start 170.85 63.625) (end 152.8225 63.625) (width 0.75) (layer "B.Cu") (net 10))
 (segment (start 153 82.725) (end 152.1 81.825) (width 0.75) (layer "B.Cu") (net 10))
 (segment (start 152.1 81.825) (end 152.1 69.5025) (width 0.75) (layer "B.Cu") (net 10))
 (segment (start 147.1 78.9) (end 147.1 78.825) (width 0.45) (layer "F.Cu") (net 22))
 (segment (start 150.2 78.9) (end 150.28 78.82) (width 0.45) (layer "F.Cu") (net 22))
 (segment (start 147.1 78.9) (end 150.2 78.9) (width 0.45) (layer "F.Cu") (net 22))
 (segment (start 172 70.425) (end 174.57 70.425) (width 0.75) (layer "F.Cu") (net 17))
 (segment (start 169.8 75.845) (end 169.8 72.625) (width 0.75) (layer "F.Cu") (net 17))
 (segment (start 174.57 70.425) (end 174.6 70.395) (width 0.75) (layer "F.Cu") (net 17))
 (segment (start 167.2 68.75) (end 167.2 67.525) (width 0.75) (layer "F.Cu") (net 17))
 (segment (start 169.8 72.625) (end 172 70.425) (width 0.75) (layer "F.Cu") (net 17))
 (via micro (at 169.8 72.625) (size 0.3) (drill 0.1) (layers "F.Cu" "B.Cu") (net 17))
 (via micro (at 167.2 67.525) (size 0.3) (drill 0.1) (layers "F.Cu" "B.Cu") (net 17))
 (segment (start 167.2 71.725) (end 168.1 72.625) (width 0.75) (layer "B.Cu") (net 17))
 (segment (start 168.1 72.625) (end 169.8 72.625) (width 0.75) (layer "B.Cu") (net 17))
 (segment (start 167.2 67.525) (end 167.2 71.725) (width 0.75) (layer "B.Cu") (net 17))
 (segment (start 156.6 83.525) (end 157.5 82.625) (width 0.25) (layer "F.Cu") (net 23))
 (segment (start 153 83.525) (end 156.6 83.525) (width 0.25) (layer "F.Cu") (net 23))
 (segment (start 157.5 82.625) (end 157.5 79.225) (width 0.25) (layer "F.Cu") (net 23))
 (segment (start 152.53 84.825) (end 152.53 83.995) (width 0.25) (layer "F.Cu") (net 23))
 (segment (start 157.095 78.82) (end 155.48 78.82) (width 0.25) (layer "F.Cu") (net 23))
 (segment (start 157.5 79.225) (end 157.095 78.82) (width 0.25) (layer "F.Cu") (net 23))
 (segment (start 152.53 83.995) (end 153 83.525) (width 0.25) (layer "F.Cu") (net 23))
 (segment (start 159.83 84.925) (end 159.93 84.825) (width 0.25) (layer "F.Cu") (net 3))
 (segment (start 155.48 80.09) (end 155.545 80.025) (width 0.25) (layer "F.Cu") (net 3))
 (segment (start 155.545 80.025) (end 156.8 80.025) (width 0.25) (layer "F.Cu") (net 3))
 (segment (start 158.6 84.925) (end 159.83 84.925) (width 0.25) (layer "F.Cu") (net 3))
 (via micro (at 156.8 80.025) (size 0.3) (drill 0.1) (layers "F.Cu" "B.Cu") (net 3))
 (via micro (at 158.6 84.925) (size 0.3) (drill 0.1) (layers "F.Cu" "B.Cu") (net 3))
 (segment (start 157.8 81.025) (end 157.8 84.725) (width 0.25) (layer "B.Cu") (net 3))
 (segment (start 157.8 84.725) (end 158 84.925) (width 0.25) (layer "B.Cu") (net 3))
 (segment (start 156.8 80.025) (end 157.8 81.025) (width 0.25) (layer "B.Cu") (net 3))
 (segment (start 158 84.925) (end 158.6 84.925) (width 0.25) (layer "B.Cu") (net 3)))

